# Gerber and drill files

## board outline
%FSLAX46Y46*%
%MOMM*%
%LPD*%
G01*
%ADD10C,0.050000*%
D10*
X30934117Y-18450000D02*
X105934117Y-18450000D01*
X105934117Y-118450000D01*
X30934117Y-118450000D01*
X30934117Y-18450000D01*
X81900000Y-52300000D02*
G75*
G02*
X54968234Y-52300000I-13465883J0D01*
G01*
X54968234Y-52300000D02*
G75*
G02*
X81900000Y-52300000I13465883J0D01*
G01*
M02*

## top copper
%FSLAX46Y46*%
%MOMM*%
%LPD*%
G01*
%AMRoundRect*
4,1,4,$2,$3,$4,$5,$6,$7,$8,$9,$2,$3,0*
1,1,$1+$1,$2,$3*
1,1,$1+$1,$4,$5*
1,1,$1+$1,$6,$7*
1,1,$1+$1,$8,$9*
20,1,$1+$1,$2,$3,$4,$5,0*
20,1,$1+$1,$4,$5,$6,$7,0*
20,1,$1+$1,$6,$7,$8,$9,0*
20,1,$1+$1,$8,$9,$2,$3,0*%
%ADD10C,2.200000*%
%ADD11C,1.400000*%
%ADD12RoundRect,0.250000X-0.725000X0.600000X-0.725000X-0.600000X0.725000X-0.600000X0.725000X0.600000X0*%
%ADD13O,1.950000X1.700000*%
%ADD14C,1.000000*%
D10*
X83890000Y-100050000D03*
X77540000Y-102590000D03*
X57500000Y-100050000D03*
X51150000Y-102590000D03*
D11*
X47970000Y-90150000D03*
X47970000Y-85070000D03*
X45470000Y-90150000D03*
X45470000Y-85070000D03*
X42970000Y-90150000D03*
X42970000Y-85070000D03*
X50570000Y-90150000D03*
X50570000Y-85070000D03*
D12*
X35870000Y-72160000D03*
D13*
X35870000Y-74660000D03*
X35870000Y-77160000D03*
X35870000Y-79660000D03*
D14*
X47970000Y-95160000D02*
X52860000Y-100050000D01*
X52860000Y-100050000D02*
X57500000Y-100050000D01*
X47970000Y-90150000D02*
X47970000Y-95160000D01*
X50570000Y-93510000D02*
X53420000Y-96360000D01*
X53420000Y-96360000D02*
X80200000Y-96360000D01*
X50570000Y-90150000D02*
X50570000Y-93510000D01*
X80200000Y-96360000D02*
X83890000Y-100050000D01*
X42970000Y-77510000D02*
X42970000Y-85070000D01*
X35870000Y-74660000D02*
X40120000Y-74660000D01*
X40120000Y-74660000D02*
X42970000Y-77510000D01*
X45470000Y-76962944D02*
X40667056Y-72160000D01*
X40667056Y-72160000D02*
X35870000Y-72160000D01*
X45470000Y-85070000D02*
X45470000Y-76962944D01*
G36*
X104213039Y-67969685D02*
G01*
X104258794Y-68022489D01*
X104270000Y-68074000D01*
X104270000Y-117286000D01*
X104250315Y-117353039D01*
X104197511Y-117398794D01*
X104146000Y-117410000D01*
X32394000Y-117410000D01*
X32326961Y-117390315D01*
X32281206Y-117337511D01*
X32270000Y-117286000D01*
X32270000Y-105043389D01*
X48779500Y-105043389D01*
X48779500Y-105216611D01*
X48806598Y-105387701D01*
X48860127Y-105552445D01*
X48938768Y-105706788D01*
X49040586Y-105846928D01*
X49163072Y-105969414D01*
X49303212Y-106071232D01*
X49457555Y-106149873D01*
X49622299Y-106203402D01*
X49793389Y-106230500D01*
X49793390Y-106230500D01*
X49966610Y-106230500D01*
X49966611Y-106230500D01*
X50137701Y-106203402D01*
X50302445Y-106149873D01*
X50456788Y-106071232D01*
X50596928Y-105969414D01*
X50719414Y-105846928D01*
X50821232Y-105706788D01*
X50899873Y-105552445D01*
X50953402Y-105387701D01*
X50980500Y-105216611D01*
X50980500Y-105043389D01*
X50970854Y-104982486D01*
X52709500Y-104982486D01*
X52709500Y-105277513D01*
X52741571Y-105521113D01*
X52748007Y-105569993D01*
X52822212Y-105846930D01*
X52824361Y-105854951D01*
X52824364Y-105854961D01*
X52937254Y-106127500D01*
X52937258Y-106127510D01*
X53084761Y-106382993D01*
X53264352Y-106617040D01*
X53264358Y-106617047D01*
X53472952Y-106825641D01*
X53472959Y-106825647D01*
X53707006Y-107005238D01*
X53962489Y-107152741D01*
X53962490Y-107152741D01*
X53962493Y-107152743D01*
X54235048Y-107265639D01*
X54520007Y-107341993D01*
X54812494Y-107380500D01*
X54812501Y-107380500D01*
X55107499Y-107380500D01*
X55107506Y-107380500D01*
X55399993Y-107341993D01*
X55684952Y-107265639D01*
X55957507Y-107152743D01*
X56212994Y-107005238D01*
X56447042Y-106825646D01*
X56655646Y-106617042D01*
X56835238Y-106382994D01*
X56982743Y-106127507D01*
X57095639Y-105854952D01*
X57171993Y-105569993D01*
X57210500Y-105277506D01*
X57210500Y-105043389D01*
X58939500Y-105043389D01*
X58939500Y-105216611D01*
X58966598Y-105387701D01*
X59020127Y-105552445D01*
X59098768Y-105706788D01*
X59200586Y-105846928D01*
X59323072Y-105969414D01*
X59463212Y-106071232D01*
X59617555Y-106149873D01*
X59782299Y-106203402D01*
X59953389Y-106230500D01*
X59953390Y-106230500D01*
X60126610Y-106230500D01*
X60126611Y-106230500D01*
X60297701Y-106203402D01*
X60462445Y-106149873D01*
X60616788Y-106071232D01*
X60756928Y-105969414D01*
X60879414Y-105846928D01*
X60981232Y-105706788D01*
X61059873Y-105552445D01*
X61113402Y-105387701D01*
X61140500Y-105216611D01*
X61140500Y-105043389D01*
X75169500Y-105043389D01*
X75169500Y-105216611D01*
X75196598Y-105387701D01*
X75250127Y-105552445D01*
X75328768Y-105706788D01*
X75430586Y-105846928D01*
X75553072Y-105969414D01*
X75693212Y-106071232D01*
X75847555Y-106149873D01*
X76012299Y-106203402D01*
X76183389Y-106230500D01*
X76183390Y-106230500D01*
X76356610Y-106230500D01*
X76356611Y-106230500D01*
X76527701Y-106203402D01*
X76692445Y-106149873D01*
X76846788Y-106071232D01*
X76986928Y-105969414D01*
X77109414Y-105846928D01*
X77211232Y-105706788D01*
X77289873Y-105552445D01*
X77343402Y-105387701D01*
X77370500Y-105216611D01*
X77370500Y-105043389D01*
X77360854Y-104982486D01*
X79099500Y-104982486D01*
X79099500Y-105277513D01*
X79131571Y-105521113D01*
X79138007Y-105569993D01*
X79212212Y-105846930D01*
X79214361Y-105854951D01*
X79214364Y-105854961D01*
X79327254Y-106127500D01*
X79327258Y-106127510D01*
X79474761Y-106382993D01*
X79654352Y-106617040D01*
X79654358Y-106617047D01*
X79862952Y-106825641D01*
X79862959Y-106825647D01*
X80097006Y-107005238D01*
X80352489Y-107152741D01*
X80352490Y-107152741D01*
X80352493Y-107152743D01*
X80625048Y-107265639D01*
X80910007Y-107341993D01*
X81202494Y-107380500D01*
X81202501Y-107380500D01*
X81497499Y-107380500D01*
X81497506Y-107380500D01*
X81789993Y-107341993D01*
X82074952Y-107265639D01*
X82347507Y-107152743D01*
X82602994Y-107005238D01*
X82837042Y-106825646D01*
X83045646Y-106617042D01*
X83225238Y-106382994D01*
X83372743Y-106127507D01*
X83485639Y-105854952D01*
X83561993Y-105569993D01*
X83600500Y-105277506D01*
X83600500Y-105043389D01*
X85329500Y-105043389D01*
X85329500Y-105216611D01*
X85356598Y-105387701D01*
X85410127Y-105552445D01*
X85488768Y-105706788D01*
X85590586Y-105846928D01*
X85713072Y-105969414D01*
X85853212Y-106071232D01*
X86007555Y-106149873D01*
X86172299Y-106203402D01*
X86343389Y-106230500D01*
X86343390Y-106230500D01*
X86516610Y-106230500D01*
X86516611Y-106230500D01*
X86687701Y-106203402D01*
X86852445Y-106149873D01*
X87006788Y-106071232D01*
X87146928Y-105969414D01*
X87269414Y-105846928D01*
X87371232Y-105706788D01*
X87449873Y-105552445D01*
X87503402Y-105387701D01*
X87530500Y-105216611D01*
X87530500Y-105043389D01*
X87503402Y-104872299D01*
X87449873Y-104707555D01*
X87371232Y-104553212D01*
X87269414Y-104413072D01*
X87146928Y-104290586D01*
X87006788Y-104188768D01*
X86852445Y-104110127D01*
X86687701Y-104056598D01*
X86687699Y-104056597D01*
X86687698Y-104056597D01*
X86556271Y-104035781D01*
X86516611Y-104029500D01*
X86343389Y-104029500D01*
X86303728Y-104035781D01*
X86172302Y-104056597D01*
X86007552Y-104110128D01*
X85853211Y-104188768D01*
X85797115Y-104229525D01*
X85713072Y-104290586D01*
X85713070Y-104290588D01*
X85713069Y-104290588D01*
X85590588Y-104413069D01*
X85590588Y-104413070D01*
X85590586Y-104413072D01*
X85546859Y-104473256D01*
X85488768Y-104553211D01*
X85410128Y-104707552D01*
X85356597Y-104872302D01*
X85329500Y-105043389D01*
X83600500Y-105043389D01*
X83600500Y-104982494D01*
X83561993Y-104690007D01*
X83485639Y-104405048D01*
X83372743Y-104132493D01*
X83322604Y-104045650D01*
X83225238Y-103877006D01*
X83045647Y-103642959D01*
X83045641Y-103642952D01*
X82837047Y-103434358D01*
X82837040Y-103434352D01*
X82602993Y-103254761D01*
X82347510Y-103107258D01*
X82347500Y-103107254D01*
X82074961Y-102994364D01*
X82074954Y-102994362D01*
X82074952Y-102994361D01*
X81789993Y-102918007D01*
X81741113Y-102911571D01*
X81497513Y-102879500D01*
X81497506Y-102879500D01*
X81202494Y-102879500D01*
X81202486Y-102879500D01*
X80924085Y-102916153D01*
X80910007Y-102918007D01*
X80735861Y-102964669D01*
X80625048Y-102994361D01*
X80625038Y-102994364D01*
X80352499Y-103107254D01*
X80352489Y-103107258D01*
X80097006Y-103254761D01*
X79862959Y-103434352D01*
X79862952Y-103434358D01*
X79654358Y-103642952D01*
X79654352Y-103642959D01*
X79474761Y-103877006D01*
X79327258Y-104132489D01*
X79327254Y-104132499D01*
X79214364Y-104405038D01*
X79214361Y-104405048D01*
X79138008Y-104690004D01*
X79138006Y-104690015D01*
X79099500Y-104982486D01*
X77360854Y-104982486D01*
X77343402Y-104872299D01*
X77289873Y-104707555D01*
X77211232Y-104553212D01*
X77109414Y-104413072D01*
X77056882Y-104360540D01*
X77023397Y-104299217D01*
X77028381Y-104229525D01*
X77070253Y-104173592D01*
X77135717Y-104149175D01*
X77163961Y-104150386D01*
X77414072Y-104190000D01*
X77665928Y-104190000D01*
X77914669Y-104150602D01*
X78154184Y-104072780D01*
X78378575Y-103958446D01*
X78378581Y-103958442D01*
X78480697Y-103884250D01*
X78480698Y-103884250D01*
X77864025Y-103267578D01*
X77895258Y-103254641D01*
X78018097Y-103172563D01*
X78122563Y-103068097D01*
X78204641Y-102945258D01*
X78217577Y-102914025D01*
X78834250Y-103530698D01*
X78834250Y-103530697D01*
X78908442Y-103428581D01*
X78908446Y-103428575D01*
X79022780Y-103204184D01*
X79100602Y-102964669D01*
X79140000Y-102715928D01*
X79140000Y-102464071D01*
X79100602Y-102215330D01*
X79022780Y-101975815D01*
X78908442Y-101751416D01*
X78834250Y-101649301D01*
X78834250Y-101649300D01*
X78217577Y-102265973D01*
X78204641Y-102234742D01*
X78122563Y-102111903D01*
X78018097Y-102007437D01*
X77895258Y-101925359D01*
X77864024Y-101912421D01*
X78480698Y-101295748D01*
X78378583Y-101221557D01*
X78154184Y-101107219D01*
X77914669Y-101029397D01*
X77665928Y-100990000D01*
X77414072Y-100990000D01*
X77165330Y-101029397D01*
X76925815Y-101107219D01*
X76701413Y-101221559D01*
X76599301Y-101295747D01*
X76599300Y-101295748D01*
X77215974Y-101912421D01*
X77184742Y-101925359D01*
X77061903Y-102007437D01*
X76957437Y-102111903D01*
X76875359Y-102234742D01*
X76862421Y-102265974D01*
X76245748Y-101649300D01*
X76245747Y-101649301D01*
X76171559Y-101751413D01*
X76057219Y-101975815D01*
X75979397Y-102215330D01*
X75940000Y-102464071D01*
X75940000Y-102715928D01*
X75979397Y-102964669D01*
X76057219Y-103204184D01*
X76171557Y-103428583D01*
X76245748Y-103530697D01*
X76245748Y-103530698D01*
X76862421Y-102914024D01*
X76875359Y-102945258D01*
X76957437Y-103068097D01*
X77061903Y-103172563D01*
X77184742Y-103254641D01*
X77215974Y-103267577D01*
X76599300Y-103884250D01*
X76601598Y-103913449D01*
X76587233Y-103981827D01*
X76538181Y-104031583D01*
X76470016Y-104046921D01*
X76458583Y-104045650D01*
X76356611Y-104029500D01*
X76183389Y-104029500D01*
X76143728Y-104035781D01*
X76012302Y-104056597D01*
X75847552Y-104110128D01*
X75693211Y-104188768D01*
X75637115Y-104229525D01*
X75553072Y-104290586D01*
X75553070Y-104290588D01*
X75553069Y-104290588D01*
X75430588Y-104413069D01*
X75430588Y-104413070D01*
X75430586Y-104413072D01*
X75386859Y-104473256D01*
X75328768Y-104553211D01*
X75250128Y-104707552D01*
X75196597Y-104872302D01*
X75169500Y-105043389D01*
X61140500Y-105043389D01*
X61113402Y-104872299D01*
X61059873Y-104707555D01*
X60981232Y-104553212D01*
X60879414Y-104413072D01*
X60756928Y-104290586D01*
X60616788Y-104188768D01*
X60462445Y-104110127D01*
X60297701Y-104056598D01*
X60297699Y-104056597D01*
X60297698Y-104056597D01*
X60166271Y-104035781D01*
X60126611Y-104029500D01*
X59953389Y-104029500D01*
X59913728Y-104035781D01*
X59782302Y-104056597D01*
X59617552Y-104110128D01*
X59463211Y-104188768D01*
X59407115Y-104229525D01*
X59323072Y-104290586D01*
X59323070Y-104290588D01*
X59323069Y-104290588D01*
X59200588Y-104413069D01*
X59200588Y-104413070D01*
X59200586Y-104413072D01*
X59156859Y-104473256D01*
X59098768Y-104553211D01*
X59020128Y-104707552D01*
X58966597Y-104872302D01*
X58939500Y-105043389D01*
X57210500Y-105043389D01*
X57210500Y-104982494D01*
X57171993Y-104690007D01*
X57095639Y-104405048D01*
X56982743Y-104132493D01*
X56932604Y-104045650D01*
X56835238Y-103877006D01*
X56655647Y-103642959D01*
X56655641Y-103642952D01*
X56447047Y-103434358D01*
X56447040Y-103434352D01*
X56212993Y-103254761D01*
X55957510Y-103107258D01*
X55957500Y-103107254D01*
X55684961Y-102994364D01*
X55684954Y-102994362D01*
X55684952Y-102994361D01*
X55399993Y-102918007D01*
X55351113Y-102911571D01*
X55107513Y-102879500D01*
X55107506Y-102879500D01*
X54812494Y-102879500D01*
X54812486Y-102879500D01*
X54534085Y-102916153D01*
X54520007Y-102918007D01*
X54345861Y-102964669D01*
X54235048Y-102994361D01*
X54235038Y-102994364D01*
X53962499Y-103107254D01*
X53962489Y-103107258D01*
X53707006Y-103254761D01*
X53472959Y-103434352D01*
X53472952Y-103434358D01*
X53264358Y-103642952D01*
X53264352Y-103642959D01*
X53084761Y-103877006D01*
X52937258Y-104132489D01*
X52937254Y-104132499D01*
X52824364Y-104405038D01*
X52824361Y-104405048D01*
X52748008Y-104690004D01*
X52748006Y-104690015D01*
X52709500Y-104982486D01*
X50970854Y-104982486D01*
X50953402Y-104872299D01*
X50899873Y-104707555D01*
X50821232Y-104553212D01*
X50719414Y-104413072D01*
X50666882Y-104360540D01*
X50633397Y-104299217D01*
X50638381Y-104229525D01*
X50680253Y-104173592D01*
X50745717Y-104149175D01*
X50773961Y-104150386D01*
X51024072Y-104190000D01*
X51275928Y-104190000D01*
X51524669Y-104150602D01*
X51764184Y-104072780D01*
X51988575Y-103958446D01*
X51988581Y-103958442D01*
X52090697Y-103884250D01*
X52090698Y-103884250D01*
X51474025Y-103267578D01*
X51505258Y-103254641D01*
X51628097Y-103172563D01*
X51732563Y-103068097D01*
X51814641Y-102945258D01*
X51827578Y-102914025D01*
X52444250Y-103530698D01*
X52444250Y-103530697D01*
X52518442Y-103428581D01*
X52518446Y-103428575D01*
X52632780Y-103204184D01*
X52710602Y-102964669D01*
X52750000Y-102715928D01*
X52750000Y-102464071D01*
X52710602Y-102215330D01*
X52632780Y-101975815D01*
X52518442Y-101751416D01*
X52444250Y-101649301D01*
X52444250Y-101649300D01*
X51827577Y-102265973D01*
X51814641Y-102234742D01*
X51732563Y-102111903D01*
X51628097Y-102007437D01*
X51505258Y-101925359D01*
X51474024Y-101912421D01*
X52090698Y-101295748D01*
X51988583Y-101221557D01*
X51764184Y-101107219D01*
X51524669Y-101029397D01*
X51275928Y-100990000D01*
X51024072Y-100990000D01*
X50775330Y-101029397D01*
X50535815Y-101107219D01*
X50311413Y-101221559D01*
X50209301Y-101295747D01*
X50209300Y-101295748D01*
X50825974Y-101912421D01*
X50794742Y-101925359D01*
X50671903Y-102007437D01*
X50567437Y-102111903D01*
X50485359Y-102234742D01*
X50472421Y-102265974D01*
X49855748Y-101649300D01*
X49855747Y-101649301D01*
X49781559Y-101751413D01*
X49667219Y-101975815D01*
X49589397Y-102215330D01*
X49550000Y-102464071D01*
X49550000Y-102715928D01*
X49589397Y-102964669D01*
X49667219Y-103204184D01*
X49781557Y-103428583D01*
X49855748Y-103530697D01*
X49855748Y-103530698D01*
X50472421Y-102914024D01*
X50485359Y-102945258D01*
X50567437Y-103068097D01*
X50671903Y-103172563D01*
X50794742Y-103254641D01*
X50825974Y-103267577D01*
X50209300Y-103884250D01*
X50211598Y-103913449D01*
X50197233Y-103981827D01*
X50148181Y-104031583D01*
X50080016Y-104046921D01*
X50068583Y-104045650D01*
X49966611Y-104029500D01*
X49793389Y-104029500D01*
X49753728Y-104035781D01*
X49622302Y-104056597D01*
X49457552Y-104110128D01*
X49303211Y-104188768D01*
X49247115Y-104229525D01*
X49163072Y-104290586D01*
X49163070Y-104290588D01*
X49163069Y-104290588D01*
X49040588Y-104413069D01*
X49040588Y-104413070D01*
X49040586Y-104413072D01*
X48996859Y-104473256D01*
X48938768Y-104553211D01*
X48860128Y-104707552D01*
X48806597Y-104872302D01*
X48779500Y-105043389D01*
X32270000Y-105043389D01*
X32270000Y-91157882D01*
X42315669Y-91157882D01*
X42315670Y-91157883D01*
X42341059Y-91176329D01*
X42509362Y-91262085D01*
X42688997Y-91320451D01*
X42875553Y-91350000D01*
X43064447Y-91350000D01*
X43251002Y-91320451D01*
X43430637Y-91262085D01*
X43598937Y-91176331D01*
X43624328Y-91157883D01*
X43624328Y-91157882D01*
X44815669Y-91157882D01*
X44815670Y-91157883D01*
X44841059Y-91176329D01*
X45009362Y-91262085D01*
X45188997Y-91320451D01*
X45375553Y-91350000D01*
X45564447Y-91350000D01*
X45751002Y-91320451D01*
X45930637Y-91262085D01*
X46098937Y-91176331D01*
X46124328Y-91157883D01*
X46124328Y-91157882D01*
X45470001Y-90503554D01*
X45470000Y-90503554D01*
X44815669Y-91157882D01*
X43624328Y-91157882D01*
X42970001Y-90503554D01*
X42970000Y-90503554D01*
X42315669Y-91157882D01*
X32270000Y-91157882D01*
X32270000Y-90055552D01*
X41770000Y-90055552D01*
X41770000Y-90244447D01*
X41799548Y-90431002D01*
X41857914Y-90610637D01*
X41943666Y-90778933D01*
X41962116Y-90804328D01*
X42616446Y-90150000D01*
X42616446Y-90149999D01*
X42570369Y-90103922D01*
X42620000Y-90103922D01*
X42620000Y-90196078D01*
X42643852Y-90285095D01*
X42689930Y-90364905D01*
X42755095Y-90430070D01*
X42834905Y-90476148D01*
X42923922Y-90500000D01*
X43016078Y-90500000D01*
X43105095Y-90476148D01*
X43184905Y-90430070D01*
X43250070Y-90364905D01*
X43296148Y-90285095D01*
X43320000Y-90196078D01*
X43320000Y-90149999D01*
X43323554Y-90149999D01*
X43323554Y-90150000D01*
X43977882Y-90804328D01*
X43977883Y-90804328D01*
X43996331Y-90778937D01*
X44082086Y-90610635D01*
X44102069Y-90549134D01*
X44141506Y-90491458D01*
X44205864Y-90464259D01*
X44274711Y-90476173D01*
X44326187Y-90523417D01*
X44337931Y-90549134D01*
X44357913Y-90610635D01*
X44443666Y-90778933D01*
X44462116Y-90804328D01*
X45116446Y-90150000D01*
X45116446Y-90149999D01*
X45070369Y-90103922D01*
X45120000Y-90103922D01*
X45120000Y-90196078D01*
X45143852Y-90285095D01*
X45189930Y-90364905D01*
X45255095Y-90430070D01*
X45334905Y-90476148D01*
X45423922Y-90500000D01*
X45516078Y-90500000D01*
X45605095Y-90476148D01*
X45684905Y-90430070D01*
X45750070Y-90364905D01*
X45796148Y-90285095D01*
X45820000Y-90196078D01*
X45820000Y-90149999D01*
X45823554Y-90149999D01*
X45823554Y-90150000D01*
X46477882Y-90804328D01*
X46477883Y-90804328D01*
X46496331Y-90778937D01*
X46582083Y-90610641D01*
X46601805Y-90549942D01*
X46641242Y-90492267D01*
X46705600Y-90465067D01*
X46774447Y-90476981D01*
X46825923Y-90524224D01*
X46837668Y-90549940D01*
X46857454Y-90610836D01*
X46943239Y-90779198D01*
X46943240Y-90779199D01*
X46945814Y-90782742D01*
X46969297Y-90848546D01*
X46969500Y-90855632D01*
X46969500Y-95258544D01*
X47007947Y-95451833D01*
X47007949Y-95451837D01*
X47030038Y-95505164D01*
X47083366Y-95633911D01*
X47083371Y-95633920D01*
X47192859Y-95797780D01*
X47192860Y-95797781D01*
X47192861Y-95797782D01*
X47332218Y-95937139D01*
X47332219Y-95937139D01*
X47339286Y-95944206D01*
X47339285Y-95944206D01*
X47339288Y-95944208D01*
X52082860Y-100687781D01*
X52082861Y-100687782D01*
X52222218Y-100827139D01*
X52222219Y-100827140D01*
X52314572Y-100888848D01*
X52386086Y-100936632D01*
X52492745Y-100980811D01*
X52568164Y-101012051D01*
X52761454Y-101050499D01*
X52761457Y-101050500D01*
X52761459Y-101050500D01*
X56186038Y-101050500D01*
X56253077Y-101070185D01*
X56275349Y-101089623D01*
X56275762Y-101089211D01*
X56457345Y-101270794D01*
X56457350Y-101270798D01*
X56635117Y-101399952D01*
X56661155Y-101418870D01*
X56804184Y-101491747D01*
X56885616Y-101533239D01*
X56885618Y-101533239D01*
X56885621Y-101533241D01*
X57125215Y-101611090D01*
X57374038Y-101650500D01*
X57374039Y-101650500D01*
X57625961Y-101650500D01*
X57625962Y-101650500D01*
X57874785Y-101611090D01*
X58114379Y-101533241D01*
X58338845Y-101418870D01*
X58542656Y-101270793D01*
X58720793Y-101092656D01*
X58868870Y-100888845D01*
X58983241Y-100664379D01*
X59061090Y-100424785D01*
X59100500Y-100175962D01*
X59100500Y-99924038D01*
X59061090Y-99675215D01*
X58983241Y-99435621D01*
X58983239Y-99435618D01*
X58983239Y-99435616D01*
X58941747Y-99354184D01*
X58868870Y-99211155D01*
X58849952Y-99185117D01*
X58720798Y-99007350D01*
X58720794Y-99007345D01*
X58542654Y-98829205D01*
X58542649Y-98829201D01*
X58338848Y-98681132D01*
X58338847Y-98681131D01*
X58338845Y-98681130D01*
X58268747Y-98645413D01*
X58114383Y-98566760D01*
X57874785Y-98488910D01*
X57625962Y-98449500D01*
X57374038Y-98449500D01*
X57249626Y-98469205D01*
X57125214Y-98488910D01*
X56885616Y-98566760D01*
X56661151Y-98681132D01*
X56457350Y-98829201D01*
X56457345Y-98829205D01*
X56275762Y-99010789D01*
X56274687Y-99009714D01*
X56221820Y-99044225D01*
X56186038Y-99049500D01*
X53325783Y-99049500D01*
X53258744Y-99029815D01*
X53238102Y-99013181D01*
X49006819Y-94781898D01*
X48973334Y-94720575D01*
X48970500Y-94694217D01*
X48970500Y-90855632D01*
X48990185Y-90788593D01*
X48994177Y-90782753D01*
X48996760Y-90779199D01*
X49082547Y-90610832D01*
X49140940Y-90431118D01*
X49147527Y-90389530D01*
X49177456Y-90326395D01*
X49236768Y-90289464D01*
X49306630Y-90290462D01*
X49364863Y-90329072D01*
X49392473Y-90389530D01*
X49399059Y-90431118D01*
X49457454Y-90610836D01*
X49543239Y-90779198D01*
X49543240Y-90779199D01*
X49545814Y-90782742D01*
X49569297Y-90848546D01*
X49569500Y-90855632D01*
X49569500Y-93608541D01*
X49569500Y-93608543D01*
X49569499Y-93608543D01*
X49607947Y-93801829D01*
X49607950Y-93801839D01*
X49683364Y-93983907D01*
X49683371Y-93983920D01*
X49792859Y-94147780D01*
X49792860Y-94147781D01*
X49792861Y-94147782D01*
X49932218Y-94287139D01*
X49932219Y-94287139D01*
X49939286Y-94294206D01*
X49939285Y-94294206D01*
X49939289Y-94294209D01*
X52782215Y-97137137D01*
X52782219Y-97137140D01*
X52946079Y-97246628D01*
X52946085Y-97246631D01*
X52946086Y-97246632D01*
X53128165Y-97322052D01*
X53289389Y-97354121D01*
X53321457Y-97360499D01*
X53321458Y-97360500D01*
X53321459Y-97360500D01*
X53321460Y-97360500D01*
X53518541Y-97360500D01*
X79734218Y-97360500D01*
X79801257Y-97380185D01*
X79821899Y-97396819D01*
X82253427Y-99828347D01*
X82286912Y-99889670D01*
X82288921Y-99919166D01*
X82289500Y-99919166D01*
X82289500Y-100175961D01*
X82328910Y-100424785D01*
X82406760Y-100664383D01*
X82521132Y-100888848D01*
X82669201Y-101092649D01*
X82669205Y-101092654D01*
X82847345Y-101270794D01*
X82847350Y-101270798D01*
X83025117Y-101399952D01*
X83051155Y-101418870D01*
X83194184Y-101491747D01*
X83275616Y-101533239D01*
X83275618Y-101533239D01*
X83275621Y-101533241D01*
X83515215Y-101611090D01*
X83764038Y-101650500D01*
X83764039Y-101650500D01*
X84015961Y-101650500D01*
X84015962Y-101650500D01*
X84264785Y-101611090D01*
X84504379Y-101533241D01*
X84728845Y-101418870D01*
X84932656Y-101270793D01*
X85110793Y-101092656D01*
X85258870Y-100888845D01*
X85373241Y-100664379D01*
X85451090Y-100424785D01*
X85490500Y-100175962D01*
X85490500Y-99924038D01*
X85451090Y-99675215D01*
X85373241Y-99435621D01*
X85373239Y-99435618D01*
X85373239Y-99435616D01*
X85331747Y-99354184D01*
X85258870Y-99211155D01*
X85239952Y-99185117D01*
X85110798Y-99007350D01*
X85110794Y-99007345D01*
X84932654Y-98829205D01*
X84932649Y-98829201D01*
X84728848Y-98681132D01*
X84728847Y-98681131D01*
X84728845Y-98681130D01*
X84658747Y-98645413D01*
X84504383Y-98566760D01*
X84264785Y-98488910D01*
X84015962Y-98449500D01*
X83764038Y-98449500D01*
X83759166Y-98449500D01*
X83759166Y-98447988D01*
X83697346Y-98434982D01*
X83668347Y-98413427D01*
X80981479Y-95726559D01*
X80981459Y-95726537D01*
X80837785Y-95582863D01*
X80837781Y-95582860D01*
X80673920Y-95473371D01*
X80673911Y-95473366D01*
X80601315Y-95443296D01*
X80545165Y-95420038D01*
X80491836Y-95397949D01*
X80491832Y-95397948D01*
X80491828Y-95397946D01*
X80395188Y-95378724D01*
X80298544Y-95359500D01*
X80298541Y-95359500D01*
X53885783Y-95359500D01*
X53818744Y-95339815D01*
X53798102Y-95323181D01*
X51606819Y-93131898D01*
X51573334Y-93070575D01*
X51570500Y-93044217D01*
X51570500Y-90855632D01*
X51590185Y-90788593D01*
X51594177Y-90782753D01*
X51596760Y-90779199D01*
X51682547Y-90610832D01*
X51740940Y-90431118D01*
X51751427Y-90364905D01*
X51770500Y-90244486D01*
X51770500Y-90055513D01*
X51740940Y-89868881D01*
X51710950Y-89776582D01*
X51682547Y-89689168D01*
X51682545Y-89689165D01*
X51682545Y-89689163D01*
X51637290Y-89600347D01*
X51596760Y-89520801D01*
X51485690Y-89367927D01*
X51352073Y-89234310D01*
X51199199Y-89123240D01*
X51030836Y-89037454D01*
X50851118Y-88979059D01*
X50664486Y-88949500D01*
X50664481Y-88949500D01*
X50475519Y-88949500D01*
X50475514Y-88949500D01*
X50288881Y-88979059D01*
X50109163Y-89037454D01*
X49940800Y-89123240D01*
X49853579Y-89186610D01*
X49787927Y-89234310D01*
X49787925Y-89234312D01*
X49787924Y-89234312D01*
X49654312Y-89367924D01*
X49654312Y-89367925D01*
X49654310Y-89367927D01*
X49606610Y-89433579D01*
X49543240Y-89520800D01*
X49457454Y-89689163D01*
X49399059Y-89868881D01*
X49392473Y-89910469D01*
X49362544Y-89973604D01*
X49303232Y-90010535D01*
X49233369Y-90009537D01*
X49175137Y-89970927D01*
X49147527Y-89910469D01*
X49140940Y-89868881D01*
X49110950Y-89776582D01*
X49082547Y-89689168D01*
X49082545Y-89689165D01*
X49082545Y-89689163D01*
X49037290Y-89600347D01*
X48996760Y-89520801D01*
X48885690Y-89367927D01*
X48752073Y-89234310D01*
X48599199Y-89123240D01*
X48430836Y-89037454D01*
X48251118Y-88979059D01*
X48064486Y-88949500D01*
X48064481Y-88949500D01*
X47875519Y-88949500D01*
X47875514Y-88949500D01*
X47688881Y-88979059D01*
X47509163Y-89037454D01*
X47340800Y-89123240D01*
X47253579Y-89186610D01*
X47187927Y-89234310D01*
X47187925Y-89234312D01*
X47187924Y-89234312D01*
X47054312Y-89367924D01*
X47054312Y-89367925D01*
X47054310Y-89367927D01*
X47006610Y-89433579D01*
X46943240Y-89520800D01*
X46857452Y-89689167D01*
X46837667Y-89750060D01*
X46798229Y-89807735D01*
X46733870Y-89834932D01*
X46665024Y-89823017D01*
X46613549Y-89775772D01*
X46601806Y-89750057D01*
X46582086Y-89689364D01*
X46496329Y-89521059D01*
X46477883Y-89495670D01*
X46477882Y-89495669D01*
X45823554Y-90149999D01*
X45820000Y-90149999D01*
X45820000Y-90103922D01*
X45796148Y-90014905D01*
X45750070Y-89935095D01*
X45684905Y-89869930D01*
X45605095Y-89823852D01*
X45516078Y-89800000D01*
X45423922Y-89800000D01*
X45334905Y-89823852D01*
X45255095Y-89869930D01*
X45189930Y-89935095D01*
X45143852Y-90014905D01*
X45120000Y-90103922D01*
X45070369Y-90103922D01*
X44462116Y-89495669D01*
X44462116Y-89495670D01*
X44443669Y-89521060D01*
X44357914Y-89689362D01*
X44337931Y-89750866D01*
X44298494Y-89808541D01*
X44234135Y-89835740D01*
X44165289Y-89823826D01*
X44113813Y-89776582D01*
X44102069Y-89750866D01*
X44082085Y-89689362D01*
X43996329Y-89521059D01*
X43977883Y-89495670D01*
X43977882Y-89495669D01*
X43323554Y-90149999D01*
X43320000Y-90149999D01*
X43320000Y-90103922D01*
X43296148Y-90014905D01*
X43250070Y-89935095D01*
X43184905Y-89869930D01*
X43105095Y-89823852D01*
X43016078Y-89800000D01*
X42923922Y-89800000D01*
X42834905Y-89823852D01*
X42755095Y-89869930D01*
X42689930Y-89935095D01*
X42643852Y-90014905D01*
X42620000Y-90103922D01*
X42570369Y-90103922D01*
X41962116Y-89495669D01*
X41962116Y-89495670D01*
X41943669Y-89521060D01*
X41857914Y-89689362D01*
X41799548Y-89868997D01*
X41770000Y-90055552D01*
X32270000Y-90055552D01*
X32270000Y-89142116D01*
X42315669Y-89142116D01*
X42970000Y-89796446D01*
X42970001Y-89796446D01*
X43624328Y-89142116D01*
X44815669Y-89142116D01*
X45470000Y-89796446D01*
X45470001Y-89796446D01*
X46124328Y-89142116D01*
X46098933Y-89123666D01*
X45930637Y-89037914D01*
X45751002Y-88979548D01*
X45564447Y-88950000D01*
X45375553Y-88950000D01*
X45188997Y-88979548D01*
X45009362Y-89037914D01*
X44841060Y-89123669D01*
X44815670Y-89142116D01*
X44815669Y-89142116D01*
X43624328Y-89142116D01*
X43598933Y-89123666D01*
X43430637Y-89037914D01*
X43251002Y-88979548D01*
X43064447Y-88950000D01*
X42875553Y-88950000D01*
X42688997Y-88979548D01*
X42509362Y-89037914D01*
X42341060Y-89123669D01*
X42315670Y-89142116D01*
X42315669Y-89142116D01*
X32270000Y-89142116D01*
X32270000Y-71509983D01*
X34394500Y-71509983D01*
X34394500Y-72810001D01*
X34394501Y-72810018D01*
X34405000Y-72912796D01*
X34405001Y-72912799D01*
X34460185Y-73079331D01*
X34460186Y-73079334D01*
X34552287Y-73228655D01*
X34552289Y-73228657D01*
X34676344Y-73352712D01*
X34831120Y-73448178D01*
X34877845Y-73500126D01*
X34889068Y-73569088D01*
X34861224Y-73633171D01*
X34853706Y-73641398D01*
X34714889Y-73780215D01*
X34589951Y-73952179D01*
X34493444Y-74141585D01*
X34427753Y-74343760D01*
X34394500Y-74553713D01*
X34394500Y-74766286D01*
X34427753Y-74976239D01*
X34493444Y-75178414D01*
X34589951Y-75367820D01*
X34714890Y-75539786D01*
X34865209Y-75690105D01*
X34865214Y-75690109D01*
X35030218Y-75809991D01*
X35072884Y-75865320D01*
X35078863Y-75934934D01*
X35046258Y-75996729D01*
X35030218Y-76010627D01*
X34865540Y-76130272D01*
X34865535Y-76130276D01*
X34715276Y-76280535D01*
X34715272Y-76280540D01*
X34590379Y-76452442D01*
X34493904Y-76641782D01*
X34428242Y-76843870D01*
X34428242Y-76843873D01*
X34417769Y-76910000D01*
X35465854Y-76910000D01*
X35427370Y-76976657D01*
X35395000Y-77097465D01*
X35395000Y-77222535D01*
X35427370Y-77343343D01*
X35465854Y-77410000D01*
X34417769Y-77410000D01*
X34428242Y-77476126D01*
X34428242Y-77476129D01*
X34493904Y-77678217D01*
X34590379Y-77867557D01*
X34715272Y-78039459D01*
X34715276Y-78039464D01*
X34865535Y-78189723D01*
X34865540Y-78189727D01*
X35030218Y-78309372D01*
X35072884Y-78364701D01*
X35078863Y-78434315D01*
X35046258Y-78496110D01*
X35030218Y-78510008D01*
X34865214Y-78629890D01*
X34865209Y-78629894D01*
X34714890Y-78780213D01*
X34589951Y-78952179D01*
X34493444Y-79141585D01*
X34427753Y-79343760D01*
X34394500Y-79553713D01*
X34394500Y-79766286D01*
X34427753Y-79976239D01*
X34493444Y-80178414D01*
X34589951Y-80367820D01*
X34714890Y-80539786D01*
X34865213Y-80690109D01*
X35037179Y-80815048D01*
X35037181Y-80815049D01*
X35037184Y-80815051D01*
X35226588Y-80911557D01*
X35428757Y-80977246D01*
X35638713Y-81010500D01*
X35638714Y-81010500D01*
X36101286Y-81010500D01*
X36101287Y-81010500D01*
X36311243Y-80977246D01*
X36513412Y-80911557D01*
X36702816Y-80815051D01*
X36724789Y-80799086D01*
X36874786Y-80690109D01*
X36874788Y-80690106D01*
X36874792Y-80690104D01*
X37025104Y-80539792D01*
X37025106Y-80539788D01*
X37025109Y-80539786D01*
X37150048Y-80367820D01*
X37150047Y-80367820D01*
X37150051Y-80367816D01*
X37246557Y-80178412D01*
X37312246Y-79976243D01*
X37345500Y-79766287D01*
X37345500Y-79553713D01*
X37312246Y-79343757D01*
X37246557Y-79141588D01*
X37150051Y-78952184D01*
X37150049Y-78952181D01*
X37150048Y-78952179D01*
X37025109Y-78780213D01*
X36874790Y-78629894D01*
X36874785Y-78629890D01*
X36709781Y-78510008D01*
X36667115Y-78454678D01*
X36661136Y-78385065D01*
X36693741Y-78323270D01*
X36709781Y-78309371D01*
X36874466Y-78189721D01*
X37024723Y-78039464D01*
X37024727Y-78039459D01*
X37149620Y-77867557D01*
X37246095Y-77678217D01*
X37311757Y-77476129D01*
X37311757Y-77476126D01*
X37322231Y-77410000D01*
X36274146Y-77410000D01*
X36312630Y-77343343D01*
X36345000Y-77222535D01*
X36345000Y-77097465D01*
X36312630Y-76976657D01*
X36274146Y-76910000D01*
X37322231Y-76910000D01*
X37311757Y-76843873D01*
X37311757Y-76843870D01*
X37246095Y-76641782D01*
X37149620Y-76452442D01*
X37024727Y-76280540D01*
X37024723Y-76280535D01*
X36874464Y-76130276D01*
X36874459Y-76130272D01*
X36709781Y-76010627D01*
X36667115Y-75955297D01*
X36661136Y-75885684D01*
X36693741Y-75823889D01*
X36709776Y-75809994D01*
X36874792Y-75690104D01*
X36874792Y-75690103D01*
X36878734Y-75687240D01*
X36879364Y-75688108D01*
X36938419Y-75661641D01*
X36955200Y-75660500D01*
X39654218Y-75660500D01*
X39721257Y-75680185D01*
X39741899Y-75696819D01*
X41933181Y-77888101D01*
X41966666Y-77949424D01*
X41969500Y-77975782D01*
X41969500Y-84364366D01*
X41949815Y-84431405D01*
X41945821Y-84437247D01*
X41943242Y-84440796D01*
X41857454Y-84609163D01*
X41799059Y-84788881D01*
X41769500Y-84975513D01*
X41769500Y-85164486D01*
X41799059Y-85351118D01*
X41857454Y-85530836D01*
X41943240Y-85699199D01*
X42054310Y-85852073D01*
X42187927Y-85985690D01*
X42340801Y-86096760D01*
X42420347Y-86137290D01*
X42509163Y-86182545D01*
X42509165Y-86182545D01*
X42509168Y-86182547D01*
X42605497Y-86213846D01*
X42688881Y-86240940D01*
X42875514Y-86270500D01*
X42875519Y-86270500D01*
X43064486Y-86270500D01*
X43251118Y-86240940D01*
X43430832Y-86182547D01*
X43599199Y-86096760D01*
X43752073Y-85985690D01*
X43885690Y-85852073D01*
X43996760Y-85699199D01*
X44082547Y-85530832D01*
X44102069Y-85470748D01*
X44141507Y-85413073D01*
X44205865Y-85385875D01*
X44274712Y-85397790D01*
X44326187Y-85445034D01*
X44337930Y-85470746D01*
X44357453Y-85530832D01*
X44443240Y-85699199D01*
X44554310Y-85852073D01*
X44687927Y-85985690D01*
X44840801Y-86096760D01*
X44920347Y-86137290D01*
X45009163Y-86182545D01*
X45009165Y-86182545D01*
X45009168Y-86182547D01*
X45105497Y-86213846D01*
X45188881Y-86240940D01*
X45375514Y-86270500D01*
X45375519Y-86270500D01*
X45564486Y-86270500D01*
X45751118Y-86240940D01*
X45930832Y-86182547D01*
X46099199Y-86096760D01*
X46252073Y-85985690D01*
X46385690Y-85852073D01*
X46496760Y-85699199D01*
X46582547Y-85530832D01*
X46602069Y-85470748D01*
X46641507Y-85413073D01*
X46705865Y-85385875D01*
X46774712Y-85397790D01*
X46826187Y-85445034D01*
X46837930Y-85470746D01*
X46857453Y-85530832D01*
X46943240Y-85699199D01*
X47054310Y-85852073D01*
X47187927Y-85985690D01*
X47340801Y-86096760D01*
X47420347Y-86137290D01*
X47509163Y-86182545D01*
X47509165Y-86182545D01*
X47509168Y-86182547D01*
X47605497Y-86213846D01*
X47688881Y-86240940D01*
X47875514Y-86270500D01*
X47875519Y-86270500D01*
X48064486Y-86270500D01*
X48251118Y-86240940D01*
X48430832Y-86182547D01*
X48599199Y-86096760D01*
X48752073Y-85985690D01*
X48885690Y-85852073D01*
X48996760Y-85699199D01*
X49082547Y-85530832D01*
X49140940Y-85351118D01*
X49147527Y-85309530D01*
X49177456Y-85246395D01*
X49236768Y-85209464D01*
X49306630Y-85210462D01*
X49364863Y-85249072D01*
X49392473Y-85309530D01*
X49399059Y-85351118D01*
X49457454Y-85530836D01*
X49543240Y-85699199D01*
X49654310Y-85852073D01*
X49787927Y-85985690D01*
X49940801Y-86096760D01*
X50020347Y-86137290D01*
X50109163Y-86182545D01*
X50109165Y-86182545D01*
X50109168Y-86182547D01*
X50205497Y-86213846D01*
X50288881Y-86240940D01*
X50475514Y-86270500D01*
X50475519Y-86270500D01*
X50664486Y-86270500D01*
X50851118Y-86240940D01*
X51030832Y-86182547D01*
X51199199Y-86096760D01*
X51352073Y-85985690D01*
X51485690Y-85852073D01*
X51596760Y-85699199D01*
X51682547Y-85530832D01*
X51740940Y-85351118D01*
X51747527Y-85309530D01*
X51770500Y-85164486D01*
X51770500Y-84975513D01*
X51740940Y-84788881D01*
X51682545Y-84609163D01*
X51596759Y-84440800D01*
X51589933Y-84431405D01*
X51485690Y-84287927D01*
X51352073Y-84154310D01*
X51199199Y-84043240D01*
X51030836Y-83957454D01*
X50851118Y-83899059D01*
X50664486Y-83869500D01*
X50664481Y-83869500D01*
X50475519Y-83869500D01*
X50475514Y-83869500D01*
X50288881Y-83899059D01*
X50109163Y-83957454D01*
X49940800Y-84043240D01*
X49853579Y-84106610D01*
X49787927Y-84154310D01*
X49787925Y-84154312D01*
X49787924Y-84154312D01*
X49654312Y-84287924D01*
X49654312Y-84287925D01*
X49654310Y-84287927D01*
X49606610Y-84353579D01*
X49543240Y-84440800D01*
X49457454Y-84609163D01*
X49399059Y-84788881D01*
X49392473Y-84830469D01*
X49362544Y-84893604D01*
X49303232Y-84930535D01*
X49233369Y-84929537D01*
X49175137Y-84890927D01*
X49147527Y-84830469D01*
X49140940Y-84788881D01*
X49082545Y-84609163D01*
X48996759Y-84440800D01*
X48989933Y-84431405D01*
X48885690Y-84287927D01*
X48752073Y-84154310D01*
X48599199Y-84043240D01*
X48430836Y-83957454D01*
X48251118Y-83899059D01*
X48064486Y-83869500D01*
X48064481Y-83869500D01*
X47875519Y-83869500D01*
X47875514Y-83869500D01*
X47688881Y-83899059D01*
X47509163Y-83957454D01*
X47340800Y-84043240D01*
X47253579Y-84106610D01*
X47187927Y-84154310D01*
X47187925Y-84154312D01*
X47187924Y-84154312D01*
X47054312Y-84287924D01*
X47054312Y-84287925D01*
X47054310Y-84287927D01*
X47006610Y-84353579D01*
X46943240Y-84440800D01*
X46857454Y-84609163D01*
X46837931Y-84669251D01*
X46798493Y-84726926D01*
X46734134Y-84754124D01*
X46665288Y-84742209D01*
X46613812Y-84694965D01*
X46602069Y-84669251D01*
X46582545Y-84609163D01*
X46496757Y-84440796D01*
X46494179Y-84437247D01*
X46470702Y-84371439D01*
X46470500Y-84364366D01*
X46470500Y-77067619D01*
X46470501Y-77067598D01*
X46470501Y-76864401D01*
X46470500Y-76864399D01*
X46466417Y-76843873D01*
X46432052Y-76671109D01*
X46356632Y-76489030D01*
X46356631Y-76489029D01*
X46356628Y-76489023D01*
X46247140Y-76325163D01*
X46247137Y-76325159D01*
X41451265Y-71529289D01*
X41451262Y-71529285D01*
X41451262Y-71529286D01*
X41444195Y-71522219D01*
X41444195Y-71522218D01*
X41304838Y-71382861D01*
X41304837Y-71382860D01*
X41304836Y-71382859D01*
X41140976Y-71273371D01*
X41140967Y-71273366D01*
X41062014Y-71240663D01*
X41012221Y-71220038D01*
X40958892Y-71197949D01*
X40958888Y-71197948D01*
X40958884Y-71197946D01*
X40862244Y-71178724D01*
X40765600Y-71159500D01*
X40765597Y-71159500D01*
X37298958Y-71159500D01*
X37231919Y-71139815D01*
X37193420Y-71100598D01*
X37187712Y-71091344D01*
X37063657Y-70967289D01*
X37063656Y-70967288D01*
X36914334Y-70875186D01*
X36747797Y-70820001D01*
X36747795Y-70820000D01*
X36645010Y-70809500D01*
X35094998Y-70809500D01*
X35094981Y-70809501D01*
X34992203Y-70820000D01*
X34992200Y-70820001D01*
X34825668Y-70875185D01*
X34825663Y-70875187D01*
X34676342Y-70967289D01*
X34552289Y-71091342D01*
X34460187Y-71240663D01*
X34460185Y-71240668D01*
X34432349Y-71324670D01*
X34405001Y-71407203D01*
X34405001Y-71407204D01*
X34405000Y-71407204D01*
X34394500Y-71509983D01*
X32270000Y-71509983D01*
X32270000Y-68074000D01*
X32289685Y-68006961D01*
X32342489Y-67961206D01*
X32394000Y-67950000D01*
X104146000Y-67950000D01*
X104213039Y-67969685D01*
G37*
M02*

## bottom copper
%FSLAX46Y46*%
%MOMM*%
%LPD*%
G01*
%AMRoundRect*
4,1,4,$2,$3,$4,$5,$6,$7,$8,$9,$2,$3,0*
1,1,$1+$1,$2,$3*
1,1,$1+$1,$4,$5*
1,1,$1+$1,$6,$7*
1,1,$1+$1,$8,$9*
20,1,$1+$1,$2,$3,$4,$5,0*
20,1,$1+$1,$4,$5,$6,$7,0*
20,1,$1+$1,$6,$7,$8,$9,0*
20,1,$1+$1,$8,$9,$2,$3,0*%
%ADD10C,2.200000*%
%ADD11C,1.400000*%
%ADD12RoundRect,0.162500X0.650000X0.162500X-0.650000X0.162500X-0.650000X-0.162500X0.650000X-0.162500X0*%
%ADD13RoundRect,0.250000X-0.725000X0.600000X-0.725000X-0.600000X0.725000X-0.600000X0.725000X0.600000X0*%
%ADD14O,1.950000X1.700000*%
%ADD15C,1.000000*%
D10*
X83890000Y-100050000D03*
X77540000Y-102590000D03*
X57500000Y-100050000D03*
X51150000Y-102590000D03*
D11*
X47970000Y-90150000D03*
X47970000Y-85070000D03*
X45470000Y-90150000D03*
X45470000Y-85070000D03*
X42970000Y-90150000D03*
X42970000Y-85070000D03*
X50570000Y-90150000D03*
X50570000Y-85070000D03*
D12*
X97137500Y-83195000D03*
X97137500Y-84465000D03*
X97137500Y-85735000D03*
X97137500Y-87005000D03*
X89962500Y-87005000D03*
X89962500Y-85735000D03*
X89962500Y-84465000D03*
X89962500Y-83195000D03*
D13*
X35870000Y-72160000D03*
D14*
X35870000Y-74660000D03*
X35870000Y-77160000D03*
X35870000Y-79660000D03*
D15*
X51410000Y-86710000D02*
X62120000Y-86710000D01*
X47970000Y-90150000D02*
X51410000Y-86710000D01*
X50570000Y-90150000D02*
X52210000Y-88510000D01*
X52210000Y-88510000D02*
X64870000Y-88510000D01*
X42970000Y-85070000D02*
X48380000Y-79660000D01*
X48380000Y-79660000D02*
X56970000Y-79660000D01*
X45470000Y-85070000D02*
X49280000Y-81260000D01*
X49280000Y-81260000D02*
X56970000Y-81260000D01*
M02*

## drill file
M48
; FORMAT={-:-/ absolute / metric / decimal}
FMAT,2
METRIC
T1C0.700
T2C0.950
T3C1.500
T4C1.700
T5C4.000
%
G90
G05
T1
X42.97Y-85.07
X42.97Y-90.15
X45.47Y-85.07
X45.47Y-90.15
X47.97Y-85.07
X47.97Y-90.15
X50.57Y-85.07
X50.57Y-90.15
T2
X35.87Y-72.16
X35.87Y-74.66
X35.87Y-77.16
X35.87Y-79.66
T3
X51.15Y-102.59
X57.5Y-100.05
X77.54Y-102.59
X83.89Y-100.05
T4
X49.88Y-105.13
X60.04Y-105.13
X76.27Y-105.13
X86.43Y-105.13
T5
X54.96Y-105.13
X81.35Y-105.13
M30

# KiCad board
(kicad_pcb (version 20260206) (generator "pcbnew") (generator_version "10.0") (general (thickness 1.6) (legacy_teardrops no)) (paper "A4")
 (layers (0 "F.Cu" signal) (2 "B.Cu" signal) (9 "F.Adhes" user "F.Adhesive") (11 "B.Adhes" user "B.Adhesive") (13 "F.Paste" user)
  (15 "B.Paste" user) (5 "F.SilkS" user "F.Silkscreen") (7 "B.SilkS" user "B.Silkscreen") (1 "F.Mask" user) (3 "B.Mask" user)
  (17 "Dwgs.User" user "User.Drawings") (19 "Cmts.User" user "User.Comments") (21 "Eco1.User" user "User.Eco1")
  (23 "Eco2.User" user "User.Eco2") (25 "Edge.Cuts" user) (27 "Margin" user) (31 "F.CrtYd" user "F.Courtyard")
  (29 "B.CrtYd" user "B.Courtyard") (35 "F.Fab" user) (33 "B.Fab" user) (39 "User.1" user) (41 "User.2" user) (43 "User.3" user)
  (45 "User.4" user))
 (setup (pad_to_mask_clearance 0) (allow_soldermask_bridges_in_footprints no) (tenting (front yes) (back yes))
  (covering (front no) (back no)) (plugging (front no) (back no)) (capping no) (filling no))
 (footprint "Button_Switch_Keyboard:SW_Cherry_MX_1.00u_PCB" (layer "F.Cu") (at 83.89 100.05)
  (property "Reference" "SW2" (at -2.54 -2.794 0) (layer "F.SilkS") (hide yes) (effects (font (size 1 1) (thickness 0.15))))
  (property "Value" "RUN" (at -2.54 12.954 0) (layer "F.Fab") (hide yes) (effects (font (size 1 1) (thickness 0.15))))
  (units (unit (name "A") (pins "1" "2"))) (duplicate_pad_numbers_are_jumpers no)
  (pad "" np_thru_hole circle (at -7.62 5.08) (size 1.7 1.7) (drill 1.7) (layers "*.Cu" "*.Mask"))
  (pad "" np_thru_hole circle (at -2.54 5.08) (size 4 4) (drill 4) (layers "*.Cu" "*.Mask"))
  (pad "" np_thru_hole circle (at 2.54 5.08) (size 1.7 1.7) (drill 1.7) (layers "*.Cu" "*.Mask"))
  (pad "1" thru_hole circle (at 0 0) (size 2.2 2.2) (drill 1.5) (layers "*.Cu" "*.Mask") (remove_unused_layers no) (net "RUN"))
  (pad "2" thru_hole circle (at -6.35 2.54) (size 2.2 2.2) (drill 1.5) (layers "*.Cu" "*.Mask") (remove_unused_layers no) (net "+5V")))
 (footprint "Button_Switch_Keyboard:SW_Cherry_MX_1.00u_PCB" (layer "F.Cu") (at 57.5 100.05)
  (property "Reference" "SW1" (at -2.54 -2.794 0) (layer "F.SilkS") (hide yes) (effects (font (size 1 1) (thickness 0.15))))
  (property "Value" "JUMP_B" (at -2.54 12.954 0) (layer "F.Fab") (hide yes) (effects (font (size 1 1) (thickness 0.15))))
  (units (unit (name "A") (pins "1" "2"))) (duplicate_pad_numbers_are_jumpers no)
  (pad "" np_thru_hole circle (at -7.62 5.08) (size 1.7 1.7) (drill 1.7) (layers "*.Cu" "*.Mask"))
  (pad "" np_thru_hole circle (at -2.54 5.08) (size 4 4) (drill 4) (layers "*.Cu" "*.Mask"))
  (pad "" np_thru_hole circle (at 2.54 5.08) (size 1.7 1.7) (drill 1.7) (layers "*.Cu" "*.Mask"))
  (pad "1" thru_hole circle (at 0 0) (size 2.2 2.2) (drill 1.5) (layers "*.Cu" "*.Mask") (remove_unused_layers no) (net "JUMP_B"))
  (pad "2" thru_hole circle (at -6.35 2.54) (size 2.2 2.2) (drill 1.5) (layers "*.Cu" "*.Mask") (remove_unused_layers no) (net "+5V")))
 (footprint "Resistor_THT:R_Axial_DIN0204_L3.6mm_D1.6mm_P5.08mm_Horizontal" (layer "F.Cu") (at 47.97 90.15 90)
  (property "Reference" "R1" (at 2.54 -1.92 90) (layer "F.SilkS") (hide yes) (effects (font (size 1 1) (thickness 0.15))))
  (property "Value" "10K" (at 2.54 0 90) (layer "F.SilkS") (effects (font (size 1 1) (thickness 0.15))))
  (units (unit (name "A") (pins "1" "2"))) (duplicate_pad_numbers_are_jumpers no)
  (pad "1" thru_hole circle (at 0 0 90) (size 1.4 1.4) (drill 0.7) (layers "*.Cu" "*.Mask") (remove_unused_layers no) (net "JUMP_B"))
  (pad "2" thru_hole circle (at 5.08 0 90) (size 1.4 1.4) (drill 0.7) (layers "*.Cu" "*.Mask") (remove_unused_layers no) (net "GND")))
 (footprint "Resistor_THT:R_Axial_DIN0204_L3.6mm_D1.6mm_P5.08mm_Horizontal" (layer "F.Cu") (at 45.47 90.15 90)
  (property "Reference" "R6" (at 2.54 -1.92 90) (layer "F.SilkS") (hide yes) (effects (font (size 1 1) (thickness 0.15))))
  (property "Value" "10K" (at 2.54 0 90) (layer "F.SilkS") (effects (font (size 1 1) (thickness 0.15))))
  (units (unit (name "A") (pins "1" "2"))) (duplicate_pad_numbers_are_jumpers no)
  (pad "1" thru_hole circle (at 0 0 90) (size 1.4 1.4) (drill 0.7) (layers "*.Cu" "*.Mask") (remove_unused_layers no) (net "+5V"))
  (pad "2" thru_hole circle (at 5.08 0 90) (size 1.4 1.4) (drill 0.7) (layers "*.Cu" "*.Mask") (remove_unused_layers no) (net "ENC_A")))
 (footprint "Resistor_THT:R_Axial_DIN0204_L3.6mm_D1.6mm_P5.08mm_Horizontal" (layer "F.Cu") (at 42.97 90.15 90)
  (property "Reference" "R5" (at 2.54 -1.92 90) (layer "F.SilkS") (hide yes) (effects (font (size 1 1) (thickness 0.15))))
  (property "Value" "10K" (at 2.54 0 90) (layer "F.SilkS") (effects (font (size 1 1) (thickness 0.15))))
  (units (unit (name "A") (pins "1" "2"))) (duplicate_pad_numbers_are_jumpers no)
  (pad "1" thru_hole circle (at 0 0 90) (size 1.4 1.4) (drill 0.7) (layers "*.Cu" "*.Mask") (remove_unused_layers no) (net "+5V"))
  (pad "2" thru_hole circle (at 5.08 0 90) (size 1.4 1.4) (drill 0.7) (layers "*.Cu" "*.Mask") (remove_unused_layers no) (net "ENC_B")))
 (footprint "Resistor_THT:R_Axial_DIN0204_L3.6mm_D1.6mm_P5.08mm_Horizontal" (layer "F.Cu") (at 50.57 90.15 90)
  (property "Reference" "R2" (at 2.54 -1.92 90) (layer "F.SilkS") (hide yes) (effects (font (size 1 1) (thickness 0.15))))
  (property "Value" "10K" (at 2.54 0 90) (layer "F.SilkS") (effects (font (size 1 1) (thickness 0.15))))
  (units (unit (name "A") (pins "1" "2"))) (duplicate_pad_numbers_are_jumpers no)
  (pad "1" thru_hole circle (at 0 0 90) (size 1.4 1.4) (drill 0.7) (layers "*.Cu" "*.Mask") (remove_unused_layers no) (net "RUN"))
  (pad "2" thru_hole circle (at 5.08 0 90) (size 1.4 1.4) (drill 0.7) (layers "*.Cu" "*.Mask") (remove_unused_layers no) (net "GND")))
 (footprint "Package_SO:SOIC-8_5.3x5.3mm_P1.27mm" (layer "B.Cu") (at 93.55 85.1 180)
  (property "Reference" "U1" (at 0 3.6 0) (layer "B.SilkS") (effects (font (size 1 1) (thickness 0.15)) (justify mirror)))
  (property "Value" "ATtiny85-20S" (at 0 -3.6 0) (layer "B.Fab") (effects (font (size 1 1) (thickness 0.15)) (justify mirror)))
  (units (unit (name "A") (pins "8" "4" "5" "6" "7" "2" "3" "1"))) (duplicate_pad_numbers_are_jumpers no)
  (pad "1" smd roundrect (at -3.5875 1.905 180) (size 1.625 0.65) (layers "B.Cu" "B.Mask" "B.Paste") (roundrect_rratio 0.25) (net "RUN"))
  (pad "2" smd roundrect (at -3.5875 0.635 180) (size 1.625 0.65) (layers "B.Cu" "B.Mask" "B.Paste") (roundrect_rratio 0.25)
   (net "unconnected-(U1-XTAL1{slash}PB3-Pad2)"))
  (pad "3" smd roundrect (at -3.5875 -0.635 180) (size 1.625 0.65) (layers "B.Cu" "B.Mask" "B.Paste") (roundrect_rratio 0.25)
   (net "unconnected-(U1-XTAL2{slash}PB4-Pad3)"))
  (pad "4" smd roundrect (at -3.5875 -1.905 180) (size 1.625 0.65) (layers "B.Cu" "B.Mask" "B.Paste") (roundrect_rratio 0.25) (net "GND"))
  (pad "5" smd roundrect (at 3.5875 -1.905 180) (size 1.625 0.65) (layers "B.Cu" "B.Mask" "B.Paste") (roundrect_rratio 0.25) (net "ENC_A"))
  (pad "6" smd roundrect (at 3.5875 -0.635 180) (size 1.625 0.65) (layers "B.Cu" "B.Mask" "B.Paste") (roundrect_rratio 0.25) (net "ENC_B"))
  (pad "7" smd roundrect (at 3.5875 0.635 180) (size 1.625 0.65) (layers "B.Cu" "B.Mask" "B.Paste") (roundrect_rratio 0.25) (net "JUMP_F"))
  (pad "8" smd roundrect (at 3.5875 1.905 180) (size 1.625 0.65) (layers "B.Cu" "B.Mask" "B.Paste") (roundrect_rratio 0.25) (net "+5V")))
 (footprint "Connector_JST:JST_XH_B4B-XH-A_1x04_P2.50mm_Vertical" (layer "B.Cu") (at 35.87 72.16 -90)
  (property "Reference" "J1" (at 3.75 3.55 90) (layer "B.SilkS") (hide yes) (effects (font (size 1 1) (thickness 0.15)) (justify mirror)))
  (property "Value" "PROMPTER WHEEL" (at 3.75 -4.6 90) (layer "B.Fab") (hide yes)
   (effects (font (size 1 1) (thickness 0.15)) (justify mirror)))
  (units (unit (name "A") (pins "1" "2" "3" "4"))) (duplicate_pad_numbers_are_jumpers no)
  (pad "1" thru_hole roundrect (at 0 0 270) (size 1.7 1.95) (drill 0.95) (layers "*.Cu" "*.Mask") (remove_unused_layers no)
   (roundrect_rratio 0.147059) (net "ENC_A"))
  (pad "2" thru_hole oval (at 2.5 0 270) (size 1.7 1.95) (drill 0.95) (layers "*.Cu" "*.Mask") (remove_unused_layers no) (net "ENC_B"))
  (pad "3" thru_hole oval (at 5 0 270) (size 1.7 1.95) (drill 0.95) (layers "*.Cu" "*.Mask") (remove_unused_layers no) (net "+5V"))
  (pad "4" thru_hole oval (at 7.5 0 270) (size 1.7 1.95) (drill 0.95) (layers "*.Cu" "*.Mask") (remove_unused_layers no) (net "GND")))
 (gr_rect (start 30.934117 18.45) (end 105.934117 118.45) (stroke (width 0.05) (type solid)) (fill no) (layer "Edge.Cuts"))
 (gr_circle (center 68.434117 52.3) (end 80.634117 58) (stroke (width 0.05) (type default)) (fill no) (layer "Edge.Cuts"))
 (segment (start 47.97 95.16) (end 52.86 100.05) (width 1) (layer "F.Cu") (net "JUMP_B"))
 (segment (start 52.86 100.05) (end 57.5 100.05) (width 1) (layer "F.Cu") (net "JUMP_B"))
 (segment (start 47.97 90.15) (end 47.97 95.16) (width 1) (layer "F.Cu") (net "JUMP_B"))
 (segment (start 51.41 86.71) (end 62.12 86.71) (width 1) (layer "B.Cu") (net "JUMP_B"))
 (segment (start 47.97 90.15) (end 51.41 86.71) (width 1) (layer "B.Cu") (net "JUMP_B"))
 (segment (start 50.57 93.51) (end 53.42 96.36) (width 1) (layer "F.Cu") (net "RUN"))
 (segment (start 53.42 96.36) (end 80.2 96.36) (width 1) (layer "F.Cu") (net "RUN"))
 (segment (start 50.57 90.15) (end 50.57 93.51) (width 1) (layer "F.Cu") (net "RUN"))
 (segment (start 80.2 96.36) (end 83.89 100.05) (width 1) (layer "F.Cu") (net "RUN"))
 (segment (start 50.57 90.15) (end 52.21 88.51) (width 1) (layer "B.Cu") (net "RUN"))
 (segment (start 52.21 88.51) (end 64.87 88.51) (width 1) (layer "B.Cu") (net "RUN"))
 (segment (start 42.97 77.51) (end 42.97 85.07) (width 1) (layer "F.Cu") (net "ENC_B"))
 (segment (start 35.87 74.66) (end 40.12 74.66) (width 1) (layer "F.Cu") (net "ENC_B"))
 (segment (start 40.12 74.66) (end 42.97 77.51) (width 1) (layer "F.Cu") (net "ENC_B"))
 (segment (start 42.97 85.07) (end 48.38 79.66) (width 1) (layer "B.Cu") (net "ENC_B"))
 (segment (start 48.38 79.66) (end 56.97 79.66) (width 1) (layer "B.Cu") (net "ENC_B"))
 (segment (start 45.47 76.962944) (end 40.667056 72.16) (width 1) (layer "F.Cu") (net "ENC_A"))
 (segment (start 40.667056 72.16) (end 35.87 72.16) (width 1) (layer "F.Cu") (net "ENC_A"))
 (segment (start 45.47 85.07) (end 45.47 76.962944) (width 1) (layer "F.Cu") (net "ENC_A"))
 (segment (start 45.47 85.07) (end 49.28 81.26) (width 1) (layer "B.Cu") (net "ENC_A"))
 (segment (start 49.28 81.26) (end 56.97 81.26) (width 1) (layer "B.Cu") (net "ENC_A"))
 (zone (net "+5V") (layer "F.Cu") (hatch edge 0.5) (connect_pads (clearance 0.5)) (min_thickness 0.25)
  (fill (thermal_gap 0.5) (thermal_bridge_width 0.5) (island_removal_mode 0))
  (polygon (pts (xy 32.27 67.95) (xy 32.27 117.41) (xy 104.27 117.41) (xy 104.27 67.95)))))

